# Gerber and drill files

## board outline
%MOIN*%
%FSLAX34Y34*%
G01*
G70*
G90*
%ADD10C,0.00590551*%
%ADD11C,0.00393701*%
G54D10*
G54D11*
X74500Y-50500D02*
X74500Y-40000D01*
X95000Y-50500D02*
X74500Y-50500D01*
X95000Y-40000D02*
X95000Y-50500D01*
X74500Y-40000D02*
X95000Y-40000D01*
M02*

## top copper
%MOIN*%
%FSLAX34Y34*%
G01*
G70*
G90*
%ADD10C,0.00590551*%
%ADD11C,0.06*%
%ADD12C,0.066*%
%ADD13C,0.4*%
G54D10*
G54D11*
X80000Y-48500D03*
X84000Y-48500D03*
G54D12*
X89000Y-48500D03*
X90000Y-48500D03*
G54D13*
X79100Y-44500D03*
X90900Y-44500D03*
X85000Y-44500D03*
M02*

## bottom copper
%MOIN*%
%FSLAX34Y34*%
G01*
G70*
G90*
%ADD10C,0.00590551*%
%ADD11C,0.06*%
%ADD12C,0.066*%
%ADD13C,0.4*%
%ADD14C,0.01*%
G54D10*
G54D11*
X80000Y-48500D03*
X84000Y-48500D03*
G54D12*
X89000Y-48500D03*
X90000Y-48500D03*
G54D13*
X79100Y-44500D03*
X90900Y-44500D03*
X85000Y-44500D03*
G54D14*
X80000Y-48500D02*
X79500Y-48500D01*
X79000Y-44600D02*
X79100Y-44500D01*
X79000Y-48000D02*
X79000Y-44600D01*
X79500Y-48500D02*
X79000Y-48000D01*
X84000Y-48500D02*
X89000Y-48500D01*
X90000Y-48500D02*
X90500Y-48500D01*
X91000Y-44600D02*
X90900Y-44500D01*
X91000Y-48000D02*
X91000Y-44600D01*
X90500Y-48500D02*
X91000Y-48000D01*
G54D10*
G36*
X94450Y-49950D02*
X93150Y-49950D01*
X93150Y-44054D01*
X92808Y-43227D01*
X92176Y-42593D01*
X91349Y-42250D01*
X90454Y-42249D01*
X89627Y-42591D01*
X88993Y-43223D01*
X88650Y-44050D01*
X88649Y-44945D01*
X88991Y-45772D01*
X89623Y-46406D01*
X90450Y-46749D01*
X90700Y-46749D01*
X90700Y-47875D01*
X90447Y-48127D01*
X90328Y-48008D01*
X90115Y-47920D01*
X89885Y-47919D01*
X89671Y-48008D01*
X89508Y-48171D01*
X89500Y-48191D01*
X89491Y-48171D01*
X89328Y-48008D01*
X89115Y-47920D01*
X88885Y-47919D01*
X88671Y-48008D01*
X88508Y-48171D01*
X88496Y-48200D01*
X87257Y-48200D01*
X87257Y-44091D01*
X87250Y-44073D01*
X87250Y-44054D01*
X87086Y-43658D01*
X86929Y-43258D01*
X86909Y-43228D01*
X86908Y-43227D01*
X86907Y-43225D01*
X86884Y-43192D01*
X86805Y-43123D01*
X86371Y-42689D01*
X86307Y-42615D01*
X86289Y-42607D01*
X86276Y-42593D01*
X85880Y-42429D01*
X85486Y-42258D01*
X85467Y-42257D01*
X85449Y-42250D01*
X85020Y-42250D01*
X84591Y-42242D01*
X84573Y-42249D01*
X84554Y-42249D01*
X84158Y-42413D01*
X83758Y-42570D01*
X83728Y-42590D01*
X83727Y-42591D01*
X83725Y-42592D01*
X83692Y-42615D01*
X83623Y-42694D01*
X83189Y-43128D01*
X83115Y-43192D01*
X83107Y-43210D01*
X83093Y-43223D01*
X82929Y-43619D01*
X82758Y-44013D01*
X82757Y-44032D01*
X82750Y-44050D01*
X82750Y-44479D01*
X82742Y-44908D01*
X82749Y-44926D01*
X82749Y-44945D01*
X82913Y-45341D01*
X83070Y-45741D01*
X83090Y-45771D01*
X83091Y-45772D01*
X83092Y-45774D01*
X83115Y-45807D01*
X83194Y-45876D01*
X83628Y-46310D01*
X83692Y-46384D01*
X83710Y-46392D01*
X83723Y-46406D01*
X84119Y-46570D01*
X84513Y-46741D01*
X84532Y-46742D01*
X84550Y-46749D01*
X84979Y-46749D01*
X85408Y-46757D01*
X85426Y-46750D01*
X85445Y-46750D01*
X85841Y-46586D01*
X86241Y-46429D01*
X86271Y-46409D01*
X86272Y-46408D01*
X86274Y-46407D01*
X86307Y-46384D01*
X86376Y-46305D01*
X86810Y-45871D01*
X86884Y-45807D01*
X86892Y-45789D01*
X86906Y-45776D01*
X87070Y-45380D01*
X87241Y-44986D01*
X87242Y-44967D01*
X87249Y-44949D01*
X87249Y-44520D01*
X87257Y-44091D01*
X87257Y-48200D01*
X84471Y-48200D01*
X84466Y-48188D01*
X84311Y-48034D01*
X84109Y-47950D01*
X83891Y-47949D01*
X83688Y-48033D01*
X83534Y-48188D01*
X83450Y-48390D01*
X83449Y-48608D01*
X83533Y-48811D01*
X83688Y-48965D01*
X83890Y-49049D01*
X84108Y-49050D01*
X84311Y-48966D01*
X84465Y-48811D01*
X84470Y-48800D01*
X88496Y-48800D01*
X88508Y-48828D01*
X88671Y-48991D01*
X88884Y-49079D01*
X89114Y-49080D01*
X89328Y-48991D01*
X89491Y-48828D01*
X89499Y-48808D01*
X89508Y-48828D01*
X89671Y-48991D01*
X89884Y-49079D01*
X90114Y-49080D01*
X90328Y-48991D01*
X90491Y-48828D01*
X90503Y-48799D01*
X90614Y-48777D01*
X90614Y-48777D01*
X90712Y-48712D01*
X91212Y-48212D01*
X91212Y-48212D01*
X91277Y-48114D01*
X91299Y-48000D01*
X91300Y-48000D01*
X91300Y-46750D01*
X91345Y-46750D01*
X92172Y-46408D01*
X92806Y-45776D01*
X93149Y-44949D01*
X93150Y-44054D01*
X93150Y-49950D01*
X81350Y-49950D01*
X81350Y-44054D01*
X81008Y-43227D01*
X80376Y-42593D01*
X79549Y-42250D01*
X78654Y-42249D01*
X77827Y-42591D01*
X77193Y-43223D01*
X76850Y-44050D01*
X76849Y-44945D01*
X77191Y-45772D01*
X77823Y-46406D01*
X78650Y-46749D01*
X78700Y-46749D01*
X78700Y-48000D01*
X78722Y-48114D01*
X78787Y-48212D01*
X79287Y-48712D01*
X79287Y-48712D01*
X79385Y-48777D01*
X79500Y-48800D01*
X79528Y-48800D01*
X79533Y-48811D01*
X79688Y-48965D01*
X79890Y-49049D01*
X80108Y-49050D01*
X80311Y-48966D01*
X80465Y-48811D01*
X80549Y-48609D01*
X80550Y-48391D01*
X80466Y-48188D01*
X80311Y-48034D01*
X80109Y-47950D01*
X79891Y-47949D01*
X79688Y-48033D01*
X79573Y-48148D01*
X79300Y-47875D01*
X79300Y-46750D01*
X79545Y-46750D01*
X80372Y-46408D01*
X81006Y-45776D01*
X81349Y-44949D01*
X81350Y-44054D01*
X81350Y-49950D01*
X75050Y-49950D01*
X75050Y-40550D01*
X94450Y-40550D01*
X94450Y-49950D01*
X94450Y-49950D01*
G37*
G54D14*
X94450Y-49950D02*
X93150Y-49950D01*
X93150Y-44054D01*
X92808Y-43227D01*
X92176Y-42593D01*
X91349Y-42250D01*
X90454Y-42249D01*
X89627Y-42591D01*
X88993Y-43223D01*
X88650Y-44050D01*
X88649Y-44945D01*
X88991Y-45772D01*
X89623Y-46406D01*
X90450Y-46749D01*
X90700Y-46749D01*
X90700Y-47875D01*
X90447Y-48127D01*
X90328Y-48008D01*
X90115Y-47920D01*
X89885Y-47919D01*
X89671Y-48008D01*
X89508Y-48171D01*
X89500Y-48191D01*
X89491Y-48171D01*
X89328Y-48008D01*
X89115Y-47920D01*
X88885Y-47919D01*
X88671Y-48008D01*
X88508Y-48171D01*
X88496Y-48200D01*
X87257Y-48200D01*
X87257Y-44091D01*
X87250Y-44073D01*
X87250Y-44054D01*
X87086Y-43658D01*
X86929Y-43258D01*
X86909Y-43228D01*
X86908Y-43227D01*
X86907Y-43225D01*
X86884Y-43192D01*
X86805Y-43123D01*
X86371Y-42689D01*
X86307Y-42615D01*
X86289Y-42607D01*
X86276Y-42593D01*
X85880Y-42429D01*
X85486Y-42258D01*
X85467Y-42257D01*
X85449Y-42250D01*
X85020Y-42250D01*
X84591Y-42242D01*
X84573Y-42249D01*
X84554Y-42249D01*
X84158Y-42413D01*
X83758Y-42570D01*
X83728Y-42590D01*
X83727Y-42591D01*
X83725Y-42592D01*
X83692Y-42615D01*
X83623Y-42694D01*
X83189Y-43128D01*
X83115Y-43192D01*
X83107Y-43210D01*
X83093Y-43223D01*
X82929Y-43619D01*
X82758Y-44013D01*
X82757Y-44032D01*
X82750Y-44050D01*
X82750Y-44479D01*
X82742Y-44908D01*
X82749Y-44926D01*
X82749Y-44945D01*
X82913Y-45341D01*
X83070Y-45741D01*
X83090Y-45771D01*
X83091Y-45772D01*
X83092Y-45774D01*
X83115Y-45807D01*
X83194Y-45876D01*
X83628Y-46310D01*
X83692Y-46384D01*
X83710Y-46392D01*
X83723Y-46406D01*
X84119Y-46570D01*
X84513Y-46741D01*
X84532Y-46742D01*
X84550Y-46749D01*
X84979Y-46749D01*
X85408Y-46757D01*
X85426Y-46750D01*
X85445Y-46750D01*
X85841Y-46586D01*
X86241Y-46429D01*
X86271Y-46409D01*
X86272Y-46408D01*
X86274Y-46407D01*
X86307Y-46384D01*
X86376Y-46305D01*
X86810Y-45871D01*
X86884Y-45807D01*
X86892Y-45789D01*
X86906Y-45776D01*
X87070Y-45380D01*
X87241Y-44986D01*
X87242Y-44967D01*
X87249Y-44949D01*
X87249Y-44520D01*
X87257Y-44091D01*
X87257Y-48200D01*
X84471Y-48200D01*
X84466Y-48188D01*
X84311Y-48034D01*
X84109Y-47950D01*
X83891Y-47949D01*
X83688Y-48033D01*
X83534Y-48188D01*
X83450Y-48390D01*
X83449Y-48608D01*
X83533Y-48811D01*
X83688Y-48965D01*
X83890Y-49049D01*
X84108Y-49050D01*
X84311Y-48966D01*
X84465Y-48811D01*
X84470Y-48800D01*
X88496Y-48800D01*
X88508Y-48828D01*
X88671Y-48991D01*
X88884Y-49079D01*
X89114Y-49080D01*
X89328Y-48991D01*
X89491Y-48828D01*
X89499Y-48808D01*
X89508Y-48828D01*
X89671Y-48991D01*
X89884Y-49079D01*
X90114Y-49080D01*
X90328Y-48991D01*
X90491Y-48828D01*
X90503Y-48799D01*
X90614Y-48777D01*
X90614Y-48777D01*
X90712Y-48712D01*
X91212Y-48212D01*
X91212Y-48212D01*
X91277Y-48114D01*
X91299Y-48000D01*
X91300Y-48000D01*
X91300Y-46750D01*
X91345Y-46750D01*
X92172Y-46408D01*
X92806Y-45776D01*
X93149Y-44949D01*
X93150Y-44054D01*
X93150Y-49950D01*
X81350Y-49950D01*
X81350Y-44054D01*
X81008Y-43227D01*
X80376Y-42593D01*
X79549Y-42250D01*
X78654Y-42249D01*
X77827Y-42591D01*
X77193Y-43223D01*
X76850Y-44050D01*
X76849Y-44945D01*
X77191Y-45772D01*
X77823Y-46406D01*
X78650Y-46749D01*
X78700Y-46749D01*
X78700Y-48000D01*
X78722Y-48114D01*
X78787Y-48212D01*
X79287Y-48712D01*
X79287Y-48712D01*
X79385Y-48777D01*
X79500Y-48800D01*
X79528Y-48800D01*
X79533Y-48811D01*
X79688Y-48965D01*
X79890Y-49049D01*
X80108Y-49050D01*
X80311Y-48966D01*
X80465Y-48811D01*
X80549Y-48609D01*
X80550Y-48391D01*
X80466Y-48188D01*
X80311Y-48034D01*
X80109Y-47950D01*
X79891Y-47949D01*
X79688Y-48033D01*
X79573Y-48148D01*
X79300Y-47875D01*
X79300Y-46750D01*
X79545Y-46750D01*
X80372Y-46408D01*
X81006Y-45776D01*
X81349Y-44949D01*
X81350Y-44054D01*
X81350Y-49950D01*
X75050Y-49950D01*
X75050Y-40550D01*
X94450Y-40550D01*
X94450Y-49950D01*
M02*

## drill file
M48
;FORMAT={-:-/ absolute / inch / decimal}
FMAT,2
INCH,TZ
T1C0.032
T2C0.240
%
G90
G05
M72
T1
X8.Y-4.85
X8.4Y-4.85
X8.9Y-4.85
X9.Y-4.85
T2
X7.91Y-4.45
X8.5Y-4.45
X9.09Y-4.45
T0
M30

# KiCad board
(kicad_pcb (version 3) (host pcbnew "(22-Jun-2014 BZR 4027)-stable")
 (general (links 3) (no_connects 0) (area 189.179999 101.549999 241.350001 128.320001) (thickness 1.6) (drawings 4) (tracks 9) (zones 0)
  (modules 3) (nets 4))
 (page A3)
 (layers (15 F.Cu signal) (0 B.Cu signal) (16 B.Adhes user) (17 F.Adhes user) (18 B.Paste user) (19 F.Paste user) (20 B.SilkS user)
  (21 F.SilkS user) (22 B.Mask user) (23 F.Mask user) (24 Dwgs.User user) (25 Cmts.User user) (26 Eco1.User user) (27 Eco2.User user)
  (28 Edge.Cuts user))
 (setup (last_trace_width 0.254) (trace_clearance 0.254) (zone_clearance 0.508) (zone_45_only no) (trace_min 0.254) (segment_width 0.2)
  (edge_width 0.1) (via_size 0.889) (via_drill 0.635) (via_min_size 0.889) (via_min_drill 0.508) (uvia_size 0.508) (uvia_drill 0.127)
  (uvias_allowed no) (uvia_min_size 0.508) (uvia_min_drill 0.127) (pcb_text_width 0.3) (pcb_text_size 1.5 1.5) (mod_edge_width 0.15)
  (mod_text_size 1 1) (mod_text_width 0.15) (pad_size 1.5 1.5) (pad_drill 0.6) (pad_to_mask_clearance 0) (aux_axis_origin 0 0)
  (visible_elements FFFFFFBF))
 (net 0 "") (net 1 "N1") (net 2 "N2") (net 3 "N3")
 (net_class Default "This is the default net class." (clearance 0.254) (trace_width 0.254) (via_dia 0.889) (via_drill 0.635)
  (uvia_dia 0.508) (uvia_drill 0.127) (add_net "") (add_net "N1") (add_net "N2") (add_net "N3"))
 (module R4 (layer F.Cu) (at 208.28 123.19) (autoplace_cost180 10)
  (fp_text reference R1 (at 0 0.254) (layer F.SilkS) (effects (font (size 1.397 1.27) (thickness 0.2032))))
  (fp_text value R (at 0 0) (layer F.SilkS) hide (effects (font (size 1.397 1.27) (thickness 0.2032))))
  (pad 1 thru_hole circle (at -5.08 0) (size 1.524 1.524) (drill 0.8128) (layers *.Cu *.Mask F.SilkS) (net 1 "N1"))
  (pad 2 thru_hole circle (at 5.08 0) (size 1.524 1.524) (drill 0.8128) (layers *.Cu *.Mask F.SilkS) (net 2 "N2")))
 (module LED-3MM (layer F.Cu) (at 227.33 123.19)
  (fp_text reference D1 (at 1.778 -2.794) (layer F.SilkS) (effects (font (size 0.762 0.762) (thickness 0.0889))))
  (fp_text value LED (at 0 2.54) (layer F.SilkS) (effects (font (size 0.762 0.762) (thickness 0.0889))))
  (pad 1 thru_hole circle (at -1.27 0) (size 1.6764 1.6764) (drill 0.8128) (layers *.Cu *.Mask F.SilkS) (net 2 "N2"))
  (pad 2 thru_hole circle (at 1.27 0) (size 1.6764 1.6764) (drill 0.8128) (layers *.Cu *.Mask F.SilkS) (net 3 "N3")))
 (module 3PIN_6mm (layer F.Cu) (at 215.9 113.03)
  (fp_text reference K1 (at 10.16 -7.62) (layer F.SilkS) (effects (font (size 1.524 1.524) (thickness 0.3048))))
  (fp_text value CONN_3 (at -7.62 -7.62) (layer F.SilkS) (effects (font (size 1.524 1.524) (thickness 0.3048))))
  (pad 1 thru_hole circle (at -14.986 0) (size 10.16 10.16) (drill 6.096) (layers *.Cu *.Mask F.SilkS) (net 1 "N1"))
  (pad 3 thru_hole circle (at 14.986 0) (size 10.16 10.16) (drill 6.096) (layers *.Cu *.Mask F.SilkS) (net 3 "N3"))
  (pad 2 thru_hole circle (at 0 0) (size 10.16 10.16) (drill 6.096) (layers *.Cu *.Mask F.SilkS)))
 (gr_line (start 189.23 128.27) (end 189.23 101.6) (angle 90) (layer Edge.Cuts) (width 0.1))
 (gr_line (start 241.3 128.27) (end 189.23 128.27) (angle 90) (layer Edge.Cuts) (width 0.1))
 (gr_line (start 241.3 101.6) (end 241.3 128.27) (angle 90) (layer Edge.Cuts) (width 0.1))
 (gr_line (start 189.23 101.6) (end 241.3 101.6) (angle 90) (layer Edge.Cuts) (width 0.1))
 (segment (start 203.2 123.19) (end 201.93 123.19) (width 0.254) (layer B.Cu) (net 1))
 (segment (start 200.66 113.284) (end 200.914 113.03) (width 0.254) (layer B.Cu) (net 1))
 (segment (start 200.66 121.92) (end 200.66 113.284) (width 0.254) (layer B.Cu) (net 1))
 (segment (start 201.93 123.19) (end 200.66 121.92) (width 0.254) (layer B.Cu) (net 1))
 (segment (start 213.36 123.19) (end 226.06 123.19) (width 0.254) (layer B.Cu) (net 2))
 (segment (start 228.6 123.19) (end 229.87 123.19) (width 0.254) (layer B.Cu) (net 3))
 (segment (start 231.14 113.284) (end 230.886 113.03) (width 0.254) (layer B.Cu) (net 3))
 (segment (start 231.14 121.92) (end 231.14 113.284) (width 0.254) (layer B.Cu) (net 3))
 (segment (start 229.87 123.19) (end 231.14 121.92) (width 0.254) (layer B.Cu) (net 3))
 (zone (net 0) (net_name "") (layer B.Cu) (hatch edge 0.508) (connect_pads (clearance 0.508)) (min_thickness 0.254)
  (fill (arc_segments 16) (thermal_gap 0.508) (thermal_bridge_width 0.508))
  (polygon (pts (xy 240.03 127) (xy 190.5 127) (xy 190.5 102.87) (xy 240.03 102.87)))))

